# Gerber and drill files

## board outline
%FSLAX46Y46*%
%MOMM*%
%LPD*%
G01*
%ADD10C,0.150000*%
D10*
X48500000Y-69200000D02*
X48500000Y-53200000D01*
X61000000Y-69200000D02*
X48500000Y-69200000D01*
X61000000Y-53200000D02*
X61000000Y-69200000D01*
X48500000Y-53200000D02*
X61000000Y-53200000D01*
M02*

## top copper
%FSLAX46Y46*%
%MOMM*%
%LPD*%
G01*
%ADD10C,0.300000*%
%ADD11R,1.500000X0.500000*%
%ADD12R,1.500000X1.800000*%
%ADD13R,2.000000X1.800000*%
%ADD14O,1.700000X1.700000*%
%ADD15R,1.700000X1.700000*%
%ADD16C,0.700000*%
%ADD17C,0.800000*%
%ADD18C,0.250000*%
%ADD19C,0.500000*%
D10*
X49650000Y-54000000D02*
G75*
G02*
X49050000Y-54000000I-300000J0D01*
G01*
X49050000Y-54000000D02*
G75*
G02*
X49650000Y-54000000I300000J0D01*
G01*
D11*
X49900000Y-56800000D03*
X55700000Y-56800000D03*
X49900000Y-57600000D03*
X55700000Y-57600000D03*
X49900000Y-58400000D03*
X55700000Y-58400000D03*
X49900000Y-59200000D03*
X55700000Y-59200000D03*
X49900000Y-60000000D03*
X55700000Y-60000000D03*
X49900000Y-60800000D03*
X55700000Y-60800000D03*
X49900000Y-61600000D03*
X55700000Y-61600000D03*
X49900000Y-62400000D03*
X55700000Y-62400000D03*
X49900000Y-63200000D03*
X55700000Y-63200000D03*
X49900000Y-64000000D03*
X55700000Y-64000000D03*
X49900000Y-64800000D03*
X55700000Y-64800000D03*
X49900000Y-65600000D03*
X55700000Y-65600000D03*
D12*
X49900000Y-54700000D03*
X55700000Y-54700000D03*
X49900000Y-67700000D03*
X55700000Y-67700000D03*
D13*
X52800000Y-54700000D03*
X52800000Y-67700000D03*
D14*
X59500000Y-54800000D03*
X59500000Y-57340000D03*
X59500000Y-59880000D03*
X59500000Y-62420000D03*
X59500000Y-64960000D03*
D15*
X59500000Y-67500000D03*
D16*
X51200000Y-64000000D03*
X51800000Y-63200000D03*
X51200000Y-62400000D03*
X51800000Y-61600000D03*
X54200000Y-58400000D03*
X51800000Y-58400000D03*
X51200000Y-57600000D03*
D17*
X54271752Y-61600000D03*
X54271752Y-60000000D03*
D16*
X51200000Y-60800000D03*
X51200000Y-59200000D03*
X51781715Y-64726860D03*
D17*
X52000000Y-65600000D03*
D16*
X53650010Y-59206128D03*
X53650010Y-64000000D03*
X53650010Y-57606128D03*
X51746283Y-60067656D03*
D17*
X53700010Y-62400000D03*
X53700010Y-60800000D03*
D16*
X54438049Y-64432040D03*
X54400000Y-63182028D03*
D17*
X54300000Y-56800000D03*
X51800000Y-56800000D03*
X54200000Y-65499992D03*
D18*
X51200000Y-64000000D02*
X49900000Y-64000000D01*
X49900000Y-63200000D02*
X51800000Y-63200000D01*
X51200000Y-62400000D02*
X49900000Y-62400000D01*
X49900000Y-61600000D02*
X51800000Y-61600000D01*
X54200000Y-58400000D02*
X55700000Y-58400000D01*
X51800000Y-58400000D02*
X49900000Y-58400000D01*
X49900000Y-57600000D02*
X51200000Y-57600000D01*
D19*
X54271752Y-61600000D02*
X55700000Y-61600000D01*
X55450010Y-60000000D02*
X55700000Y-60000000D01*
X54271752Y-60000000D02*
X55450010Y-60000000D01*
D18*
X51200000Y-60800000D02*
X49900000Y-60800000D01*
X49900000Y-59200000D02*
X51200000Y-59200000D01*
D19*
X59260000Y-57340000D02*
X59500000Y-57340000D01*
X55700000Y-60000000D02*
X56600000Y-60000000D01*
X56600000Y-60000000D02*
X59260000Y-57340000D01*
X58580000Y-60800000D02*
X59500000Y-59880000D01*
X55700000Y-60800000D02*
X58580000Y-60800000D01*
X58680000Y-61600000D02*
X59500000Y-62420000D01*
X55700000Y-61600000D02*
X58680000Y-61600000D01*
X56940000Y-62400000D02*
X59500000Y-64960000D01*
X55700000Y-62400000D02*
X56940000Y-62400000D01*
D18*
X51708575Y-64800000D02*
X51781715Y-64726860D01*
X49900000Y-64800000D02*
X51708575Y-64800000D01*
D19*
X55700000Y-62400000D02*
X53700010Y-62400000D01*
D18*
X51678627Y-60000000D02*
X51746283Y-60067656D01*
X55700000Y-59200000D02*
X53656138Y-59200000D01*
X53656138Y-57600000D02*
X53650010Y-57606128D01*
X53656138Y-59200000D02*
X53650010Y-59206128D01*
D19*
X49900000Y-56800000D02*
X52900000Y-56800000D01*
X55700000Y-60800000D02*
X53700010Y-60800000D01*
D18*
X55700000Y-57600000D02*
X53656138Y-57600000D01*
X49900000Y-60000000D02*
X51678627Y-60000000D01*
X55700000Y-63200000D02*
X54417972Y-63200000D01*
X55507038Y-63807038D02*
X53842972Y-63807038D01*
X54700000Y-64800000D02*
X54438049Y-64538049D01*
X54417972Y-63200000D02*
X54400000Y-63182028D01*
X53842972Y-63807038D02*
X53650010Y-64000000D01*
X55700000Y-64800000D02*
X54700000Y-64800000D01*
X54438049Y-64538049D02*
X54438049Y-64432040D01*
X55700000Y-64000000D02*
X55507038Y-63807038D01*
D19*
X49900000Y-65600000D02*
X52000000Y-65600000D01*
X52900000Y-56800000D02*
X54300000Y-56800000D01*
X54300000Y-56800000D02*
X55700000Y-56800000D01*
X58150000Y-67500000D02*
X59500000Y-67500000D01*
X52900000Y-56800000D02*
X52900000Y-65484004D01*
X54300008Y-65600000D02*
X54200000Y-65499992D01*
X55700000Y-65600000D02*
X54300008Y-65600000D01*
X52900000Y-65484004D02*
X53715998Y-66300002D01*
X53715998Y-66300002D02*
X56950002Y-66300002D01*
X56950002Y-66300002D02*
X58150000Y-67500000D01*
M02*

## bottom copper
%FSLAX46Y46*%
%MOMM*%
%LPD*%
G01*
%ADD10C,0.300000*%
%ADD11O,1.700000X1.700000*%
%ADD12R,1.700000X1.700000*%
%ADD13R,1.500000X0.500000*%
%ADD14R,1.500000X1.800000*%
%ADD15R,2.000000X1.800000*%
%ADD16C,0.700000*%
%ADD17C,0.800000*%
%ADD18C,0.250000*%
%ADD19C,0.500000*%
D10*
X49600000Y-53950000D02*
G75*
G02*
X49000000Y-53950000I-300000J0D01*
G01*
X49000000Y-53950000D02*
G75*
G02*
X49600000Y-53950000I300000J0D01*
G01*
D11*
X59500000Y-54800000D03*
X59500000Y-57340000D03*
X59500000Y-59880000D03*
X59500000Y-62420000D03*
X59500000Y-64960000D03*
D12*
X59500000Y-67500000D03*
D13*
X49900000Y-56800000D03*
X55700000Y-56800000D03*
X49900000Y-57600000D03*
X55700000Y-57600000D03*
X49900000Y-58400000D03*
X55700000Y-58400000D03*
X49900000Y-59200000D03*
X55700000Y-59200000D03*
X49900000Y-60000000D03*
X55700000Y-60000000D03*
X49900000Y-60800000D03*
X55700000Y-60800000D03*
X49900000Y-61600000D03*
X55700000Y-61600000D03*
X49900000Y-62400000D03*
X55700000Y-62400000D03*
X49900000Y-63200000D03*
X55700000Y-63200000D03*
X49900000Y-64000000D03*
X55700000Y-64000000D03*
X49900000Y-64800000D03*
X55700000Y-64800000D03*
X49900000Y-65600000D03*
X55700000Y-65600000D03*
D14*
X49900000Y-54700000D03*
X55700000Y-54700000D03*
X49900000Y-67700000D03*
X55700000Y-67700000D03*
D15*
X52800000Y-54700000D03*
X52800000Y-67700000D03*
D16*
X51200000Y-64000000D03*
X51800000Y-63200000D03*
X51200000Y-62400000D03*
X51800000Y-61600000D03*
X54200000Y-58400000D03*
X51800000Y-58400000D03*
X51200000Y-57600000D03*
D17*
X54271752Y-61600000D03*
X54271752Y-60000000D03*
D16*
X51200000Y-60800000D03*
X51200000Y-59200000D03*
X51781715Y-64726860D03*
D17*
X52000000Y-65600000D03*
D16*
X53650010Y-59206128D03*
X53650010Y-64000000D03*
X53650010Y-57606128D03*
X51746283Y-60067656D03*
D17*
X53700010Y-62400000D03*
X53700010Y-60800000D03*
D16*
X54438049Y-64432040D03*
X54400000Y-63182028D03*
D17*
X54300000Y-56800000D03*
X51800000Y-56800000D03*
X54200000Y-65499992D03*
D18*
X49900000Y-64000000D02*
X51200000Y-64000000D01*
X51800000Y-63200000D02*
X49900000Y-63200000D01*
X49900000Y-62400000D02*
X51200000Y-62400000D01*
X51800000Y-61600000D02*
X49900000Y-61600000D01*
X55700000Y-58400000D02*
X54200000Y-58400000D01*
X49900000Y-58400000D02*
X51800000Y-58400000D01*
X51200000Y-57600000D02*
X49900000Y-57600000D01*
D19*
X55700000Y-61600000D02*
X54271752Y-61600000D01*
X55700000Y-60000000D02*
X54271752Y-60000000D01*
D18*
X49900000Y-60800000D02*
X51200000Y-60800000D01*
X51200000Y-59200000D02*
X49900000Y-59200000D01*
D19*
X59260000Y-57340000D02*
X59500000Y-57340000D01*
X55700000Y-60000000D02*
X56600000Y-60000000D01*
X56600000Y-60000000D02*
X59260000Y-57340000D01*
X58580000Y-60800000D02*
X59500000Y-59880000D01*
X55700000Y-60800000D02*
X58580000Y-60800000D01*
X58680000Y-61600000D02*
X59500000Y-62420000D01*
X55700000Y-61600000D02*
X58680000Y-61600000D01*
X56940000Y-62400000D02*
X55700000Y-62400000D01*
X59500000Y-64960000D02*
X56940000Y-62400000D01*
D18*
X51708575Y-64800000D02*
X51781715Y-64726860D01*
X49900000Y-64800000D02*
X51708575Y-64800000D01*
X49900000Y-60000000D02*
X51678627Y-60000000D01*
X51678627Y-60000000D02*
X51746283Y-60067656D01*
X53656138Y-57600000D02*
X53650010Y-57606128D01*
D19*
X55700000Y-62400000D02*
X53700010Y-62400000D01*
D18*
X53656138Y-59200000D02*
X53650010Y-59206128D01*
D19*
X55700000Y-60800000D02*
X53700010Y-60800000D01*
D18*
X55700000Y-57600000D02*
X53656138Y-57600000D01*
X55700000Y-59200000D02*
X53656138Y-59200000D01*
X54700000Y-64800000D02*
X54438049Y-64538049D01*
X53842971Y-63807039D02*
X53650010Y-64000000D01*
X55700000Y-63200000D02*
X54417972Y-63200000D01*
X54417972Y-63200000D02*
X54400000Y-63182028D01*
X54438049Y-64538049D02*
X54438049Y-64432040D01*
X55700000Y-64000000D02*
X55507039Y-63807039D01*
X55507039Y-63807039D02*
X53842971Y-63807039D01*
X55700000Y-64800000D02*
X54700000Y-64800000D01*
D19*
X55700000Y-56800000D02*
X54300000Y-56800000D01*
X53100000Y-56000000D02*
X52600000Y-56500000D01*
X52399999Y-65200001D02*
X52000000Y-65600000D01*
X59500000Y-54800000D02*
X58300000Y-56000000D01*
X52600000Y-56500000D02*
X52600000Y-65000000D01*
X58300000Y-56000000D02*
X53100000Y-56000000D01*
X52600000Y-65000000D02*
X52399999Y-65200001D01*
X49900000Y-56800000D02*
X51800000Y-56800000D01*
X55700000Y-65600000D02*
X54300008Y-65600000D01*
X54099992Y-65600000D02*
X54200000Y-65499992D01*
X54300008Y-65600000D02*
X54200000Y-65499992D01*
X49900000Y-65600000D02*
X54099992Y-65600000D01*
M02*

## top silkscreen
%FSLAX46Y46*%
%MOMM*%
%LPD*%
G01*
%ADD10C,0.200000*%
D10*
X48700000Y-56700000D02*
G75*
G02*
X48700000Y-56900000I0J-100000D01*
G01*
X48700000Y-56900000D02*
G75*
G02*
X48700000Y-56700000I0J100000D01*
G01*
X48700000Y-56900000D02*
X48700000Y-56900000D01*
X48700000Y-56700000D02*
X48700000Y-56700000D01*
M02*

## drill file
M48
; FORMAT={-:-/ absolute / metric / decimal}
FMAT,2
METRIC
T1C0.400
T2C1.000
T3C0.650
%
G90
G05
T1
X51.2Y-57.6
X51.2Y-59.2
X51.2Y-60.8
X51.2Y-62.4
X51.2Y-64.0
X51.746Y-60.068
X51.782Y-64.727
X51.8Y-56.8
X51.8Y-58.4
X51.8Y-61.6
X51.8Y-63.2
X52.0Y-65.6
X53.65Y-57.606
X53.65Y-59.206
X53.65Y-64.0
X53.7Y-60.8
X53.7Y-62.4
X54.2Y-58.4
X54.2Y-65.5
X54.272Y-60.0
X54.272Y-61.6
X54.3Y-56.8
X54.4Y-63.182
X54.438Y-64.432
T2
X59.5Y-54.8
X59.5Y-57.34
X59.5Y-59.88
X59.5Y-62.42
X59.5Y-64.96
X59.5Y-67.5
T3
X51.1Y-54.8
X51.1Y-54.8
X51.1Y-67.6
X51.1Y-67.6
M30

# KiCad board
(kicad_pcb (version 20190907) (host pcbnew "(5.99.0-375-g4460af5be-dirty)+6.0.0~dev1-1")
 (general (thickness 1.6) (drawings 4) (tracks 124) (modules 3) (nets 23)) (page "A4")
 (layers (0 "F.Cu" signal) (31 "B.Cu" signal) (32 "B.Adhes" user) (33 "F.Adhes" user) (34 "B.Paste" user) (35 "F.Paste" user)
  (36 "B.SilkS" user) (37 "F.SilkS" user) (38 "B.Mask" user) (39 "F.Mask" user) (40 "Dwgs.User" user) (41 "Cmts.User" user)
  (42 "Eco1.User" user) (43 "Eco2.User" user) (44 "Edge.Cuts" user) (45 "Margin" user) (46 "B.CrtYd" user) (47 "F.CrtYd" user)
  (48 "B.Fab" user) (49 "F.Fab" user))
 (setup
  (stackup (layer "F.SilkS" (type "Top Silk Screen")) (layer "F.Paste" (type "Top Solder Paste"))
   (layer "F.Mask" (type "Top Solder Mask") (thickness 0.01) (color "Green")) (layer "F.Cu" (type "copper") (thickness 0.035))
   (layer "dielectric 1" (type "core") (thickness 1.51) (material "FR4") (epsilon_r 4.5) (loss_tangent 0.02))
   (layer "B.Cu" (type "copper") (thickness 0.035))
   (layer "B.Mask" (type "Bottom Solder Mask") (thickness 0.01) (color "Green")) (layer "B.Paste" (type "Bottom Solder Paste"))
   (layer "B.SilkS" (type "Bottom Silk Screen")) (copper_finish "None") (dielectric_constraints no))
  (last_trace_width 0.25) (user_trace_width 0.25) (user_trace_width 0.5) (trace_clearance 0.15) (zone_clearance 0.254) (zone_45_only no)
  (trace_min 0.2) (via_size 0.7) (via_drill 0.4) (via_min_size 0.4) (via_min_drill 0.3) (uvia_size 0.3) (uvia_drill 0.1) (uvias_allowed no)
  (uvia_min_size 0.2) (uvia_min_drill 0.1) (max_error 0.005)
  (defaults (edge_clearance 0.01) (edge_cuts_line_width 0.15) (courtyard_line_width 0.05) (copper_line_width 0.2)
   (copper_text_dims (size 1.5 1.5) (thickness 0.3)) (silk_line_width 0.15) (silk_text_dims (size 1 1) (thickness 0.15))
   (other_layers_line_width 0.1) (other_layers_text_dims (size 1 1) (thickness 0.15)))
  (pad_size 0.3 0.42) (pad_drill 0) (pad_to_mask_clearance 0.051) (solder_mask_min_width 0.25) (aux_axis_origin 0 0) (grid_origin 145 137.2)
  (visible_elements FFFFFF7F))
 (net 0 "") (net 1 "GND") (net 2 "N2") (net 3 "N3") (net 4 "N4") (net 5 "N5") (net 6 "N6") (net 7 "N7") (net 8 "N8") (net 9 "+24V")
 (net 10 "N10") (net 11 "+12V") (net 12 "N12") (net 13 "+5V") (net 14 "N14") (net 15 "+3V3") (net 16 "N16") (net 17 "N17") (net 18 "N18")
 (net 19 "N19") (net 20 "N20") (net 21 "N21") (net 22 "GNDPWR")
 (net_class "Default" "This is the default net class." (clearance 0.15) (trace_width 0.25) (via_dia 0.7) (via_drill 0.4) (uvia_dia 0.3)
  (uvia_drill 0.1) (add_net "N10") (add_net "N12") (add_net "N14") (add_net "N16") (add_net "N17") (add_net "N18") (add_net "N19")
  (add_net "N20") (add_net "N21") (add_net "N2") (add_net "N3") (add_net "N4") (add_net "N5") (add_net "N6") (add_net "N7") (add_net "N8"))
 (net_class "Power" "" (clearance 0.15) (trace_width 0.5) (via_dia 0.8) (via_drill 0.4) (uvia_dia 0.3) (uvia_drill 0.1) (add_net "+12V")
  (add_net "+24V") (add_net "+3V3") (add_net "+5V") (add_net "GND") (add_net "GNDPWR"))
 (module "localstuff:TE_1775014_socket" (layer "F.Cu") (at 52.8 61.2 -90)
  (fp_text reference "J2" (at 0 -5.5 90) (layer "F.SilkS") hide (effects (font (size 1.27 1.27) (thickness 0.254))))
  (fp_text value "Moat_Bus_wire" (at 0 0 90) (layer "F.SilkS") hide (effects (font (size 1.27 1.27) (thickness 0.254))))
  (fp_arc (start -4.4 4.1) (end -4.3 4.1) (angle -180) (layer "F.SilkS") (width 0.2))
  (fp_arc (start -4.4 4.1) (end -4.5 4.1) (angle -180) (layer "F.SilkS") (width 0.2))
  (fp_line (start -4.3 4.1) (end -4.3 4.1) (layer "F.SilkS") (width 0.2))
  (fp_line (start -4.5 4.1) (end -4.5 4.1) (layer "F.SilkS") (width 0.2))
  (fp_circle (center -7.2 3.45) (end -6.9 3.45) (layer "F.Cu") (width 0.3))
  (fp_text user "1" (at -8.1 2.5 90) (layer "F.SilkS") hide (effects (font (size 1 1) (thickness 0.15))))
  (pad "1" smd rect (at -4.4 2.9 270) (size 0.5 1.5) (layers "F.Cu" "F.Paste" "F.Mask") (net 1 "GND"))
  (pad "2" smd rect (at -4.4 -2.9 270) (size 0.5 1.5) (layers "F.Cu" "F.Paste" "F.Mask") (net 1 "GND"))
  (pad "3" smd rect (at -3.6 2.9 270) (size 0.5 1.5) (layers "F.Cu" "F.Paste" "F.Mask") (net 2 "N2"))
  (pad "4" smd rect (at -3.6 -2.9 270) (size 0.5 1.5) (layers "F.Cu" "F.Paste" "F.Mask") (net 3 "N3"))
  (pad "5" smd rect (at -2.8 2.9 270) (size 0.5 1.5) (layers "F.Cu" "F.Paste" "F.Mask") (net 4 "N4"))
  (pad "6" smd rect (at -2.8 -2.9 270) (size 0.5 1.5) (layers "F.Cu" "F.Paste" "F.Mask") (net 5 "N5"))
  (pad "7" smd rect (at -2 2.9 270) (size 0.5 1.5) (layers "F.Cu" "F.Paste" "F.Mask") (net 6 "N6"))
  (pad "8" smd rect (at -2 -2.9 270) (size 0.5 1.5) (layers "F.Cu" "F.Paste" "F.Mask") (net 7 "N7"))
  (pad "9" smd rect (at -1.2 2.9 270) (size 0.5 1.5) (layers "F.Cu" "F.Paste" "F.Mask") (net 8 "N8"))
  (pad "10" smd rect (at -1.2 -2.9 270) (size 0.5 1.5) (layers "F.Cu" "F.Paste" "F.Mask") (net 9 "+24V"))
  (pad "11" smd rect (at -0.4 2.9 270) (size 0.5 1.5) (layers "F.Cu" "F.Paste" "F.Mask") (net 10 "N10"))
  (pad "12" smd rect (at -0.4 -2.9 270) (size 0.5 1.5) (layers "F.Cu" "F.Paste" "F.Mask") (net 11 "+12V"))
  (pad "13" smd rect (at 0.4 2.9 270) (size 0.5 1.5) (layers "F.Cu" "F.Paste" "F.Mask") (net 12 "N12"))
  (pad "14" smd rect (at 0.4 -2.9 270) (size 0.5 1.5) (layers "F.Cu" "F.Paste" "F.Mask") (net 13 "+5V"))
  (pad "15" smd rect (at 1.2 2.9 270) (size 0.5 1.5) (layers "F.Cu" "F.Paste" "F.Mask") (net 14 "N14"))
  (pad "16" smd rect (at 1.2 -2.9 270) (size 0.5 1.5) (layers "F.Cu" "F.Paste" "F.Mask") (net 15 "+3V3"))
  (pad "17" smd rect (at 2 2.9 270) (size 0.5 1.5) (layers "F.Cu" "F.Paste" "F.Mask") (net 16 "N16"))
  (pad "18" smd rect (at 2 -2.9 270) (size 0.5 1.5) (layers "F.Cu" "F.Paste" "F.Mask") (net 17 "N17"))
  (pad "19" smd rect (at 2.8 2.9 270) (size 0.5 1.5) (layers "F.Cu" "F.Paste" "F.Mask") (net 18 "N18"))
  (pad "20" smd rect (at 2.8 -2.9 270) (size 0.5 1.5) (layers "F.Cu" "F.Paste" "F.Mask") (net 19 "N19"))
  (pad "21" smd rect (at 3.6 2.9 270) (size 0.5 1.5) (layers "F.Cu" "F.Paste" "F.Mask") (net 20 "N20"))
  (pad "22" smd rect (at 3.6 -2.9 270) (size 0.5 1.5) (layers "F.Cu" "F.Paste" "F.Mask") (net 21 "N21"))
  (pad "23" smd rect (at 4.4 2.9 270) (size 0.5 1.5) (layers "F.Cu" "F.Paste" "F.Mask") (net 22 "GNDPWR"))
  (pad "24" smd rect (at 4.4 -2.9 270) (size 0.5 1.5) (layers "F.Cu" "F.Paste" "F.Mask") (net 22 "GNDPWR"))
  (pad "MNT" smd rect (at -6.5 2.9) (size 1.5 1.8) (layers "F.Cu" "F.Paste" "F.Mask") (solder_paste_margin -0.05) (clearance 0.001))
  (pad "MNT" smd rect (at -6.5 -2.9) (size 1.5 1.8) (layers "F.Cu" "F.Paste" "F.Mask"))
  (pad "MNT" smd rect (at 6.5 2.9) (size 1.5 1.8) (layers "F.Cu" "F.Paste" "F.Mask") (solder_paste_margin -0.05) (clearance 0.001))
  (pad "MNT" smd rect (at 6.5 -2.9) (size 1.5 1.8) (layers "F.Cu" "F.Paste" "F.Mask"))
  (pad "MNT" smd rect (at -6.5 0 270) (size 1.8 2) (layers "F.Cu" "F.Paste" "F.Mask"))
  (pad "MNT" smd rect (at 6.5 0 270) (size 1.8 2) (layers "F.Cu" "F.Paste" "F.Mask"))
  (pad "" np_thru_hole circle (at -6.4 1.7 270) (size 0.65 0.65) (drill 0.65) (layers *.Cu *.Mask) (clearance 0.01))
  (pad "" np_thru_hole circle (at 6.4 1.7 270) (size 0.65 0.65) (drill 0.65) (layers *.Cu *.Mask) (clearance 0.0001)))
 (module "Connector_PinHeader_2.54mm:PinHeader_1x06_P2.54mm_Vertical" (layer "B.Cu") (at 59.5 67.5)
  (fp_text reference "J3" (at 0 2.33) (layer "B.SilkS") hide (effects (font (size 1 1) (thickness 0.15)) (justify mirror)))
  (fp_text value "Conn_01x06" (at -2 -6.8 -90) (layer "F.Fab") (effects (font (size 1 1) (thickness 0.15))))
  (pad "6" thru_hole oval (at 0 -12.7) (size 1.7 1.7) (drill 1) (layers *.Cu *.Mask) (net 22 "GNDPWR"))
  (pad "5" thru_hole oval (at 0 -10.16) (size 1.7 1.7) (drill 1) (layers *.Cu *.Mask) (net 9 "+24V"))
  (pad "4" thru_hole oval (at 0 -7.62) (size 1.7 1.7) (drill 1) (layers *.Cu *.Mask) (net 11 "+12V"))
  (pad "3" thru_hole oval (at 0 -5.08) (size 1.7 1.7) (drill 1) (layers *.Cu *.Mask) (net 13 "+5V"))
  (pad "2" thru_hole oval (at 0 -2.54) (size 1.7 1.7) (drill 1) (layers *.Cu *.Mask) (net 15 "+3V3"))
  (pad "1" thru_hole rect (at 0 0) (size 1.7 1.7) (drill 1) (layers *.Cu *.Mask) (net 1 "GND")))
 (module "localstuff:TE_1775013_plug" (layer "B.Cu") (at 52.8 61.2 90)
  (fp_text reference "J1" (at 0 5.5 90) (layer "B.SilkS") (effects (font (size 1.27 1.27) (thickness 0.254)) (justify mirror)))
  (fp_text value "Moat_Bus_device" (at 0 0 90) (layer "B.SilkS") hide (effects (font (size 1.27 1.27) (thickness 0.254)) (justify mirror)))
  (fp_circle (center 7.25 -3.5) (end 7.55 -3.5) (layer "B.Cu") (width 0.3))
  (pad "1" smd rect (at 4.4 -2.9 90) (size 0.5 1.5) (layers "B.Cu" "B.Paste" "B.Mask") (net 1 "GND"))
  (pad "2" smd rect (at 4.4 2.9 90) (size 0.5 1.5) (layers "B.Cu" "B.Paste" "B.Mask") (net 1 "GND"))
  (pad "3" smd rect (at 3.6 -2.9 90) (size 0.5 1.5) (layers "B.Cu" "B.Paste" "B.Mask") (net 2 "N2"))
  (pad "4" smd rect (at 3.6 2.9 90) (size 0.5 1.5) (layers "B.Cu" "B.Paste" "B.Mask") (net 3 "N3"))
  (pad "5" smd rect (at 2.8 -2.9 90) (size 0.5 1.5) (layers "B.Cu" "B.Paste" "B.Mask") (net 4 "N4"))
  (pad "6" smd rect (at 2.8 2.9 90) (size 0.5 1.5) (layers "B.Cu" "B.Paste" "B.Mask") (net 5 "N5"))
  (pad "7" smd rect (at 2 -2.9 90) (size 0.5 1.5) (layers "B.Cu" "B.Paste" "B.Mask") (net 6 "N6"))
  (pad "8" smd rect (at 2 2.9 90) (size 0.5 1.5) (layers "B.Cu" "B.Paste" "B.Mask") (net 7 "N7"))
  (pad "9" smd rect (at 1.2 -2.9 90) (size 0.5 1.5) (layers "B.Cu" "B.Paste" "B.Mask") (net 8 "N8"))
  (pad "10" smd rect (at 1.2 2.9 90) (size 0.5 1.5) (layers "B.Cu" "B.Paste" "B.Mask") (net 9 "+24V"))
  (pad "11" smd rect (at 0.4 -2.9 90) (size 0.5 1.5) (layers "B.Cu" "B.Paste" "B.Mask") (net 10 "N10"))
  (pad "12" smd rect (at 0.4 2.9 90) (size 0.5 1.5) (layers "B.Cu" "B.Paste" "B.Mask") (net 11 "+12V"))
  (pad "13" smd rect (at -0.4 -2.9 90) (size 0.5 1.5) (layers "B.Cu" "B.Paste" "B.Mask") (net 12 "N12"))
  (pad "14" smd rect (at -0.4 2.9 90) (size 0.5 1.5) (layers "B.Cu" "B.Paste" "B.Mask") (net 13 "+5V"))
  (pad "15" smd rect (at -1.2 -2.9 90) (size 0.5 1.5) (layers "B.Cu" "B.Paste" "B.Mask") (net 14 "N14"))
  (pad "16" smd rect (at -1.2 2.9 90) (size 0.5 1.5) (layers "B.Cu" "B.Paste" "B.Mask") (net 15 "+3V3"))
  (pad "17" smd rect (at -2 -2.9 90) (size 0.5 1.5) (layers "B.Cu" "B.Paste" "B.Mask") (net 16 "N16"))
  (pad "18" smd rect (at -2 2.9 90) (size 0.5 1.5) (layers "B.Cu" "B.Paste" "B.Mask") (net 17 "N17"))
  (pad "19" smd rect (at -2.8 -2.9 90) (size 0.5 1.5) (layers "B.Cu" "B.Paste" "B.Mask") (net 18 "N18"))
  (pad "20" smd rect (at -2.8 2.9 90) (size 0.5 1.5) (layers "B.Cu" "B.Paste" "B.Mask") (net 19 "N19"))
  (pad "21" smd rect (at -3.6 -2.9 90) (size 0.5 1.5) (layers "B.Cu" "B.Paste" "B.Mask") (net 20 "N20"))
  (pad "22" smd rect (at -3.6 2.9 90) (size 0.5 1.5) (layers "B.Cu" "B.Paste" "B.Mask") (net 21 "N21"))
  (pad "23" smd rect (at -4.4 -2.9 90) (size 0.5 1.5) (layers "B.Cu" "B.Paste" "B.Mask") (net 22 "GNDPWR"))
  (pad "24" smd rect (at -4.4 2.9 90) (size 0.5 1.5) (layers "B.Cu" "B.Paste" "B.Mask") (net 22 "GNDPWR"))
  (pad "MNT" smd rect (at 6.5 -2.9 180) (size 1.5 1.8) (layers "B.Cu" "B.Paste" "B.Mask"))
  (pad "MNT" smd rect (at 6.5 2.9 180) (size 1.5 1.8) (layers "B.Cu" "B.Paste" "B.Mask"))
  (pad "MNT" smd rect (at -6.5 -2.9 180) (size 1.5 1.8) (layers "B.Cu" "B.Paste" "B.Mask"))
  (pad "MNT" smd rect (at -6.5 2.9 180) (size 1.5 1.8) (layers "B.Cu" "B.Paste" "B.Mask"))
  (pad "MNT" smd rect (at 6.5 0 90) (size 1.8 2) (layers "B.Cu" "B.Paste" "B.Mask"))
  (pad "MNT" smd rect (at -6.5 0 90) (size 1.8 2) (layers "B.Cu" "B.Paste" "B.Mask"))
  (pad "" np_thru_hole circle (at 6.4 -1.7 90) (size 0.65 0.65) (drill 0.65) (layers *.Cu *.Mask))
  (pad "" np_thru_hole circle (at -6.4 -1.7 90) (size 0.65 0.65) (drill 0.65) (layers *.Cu *.Mask)))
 (gr_line (start 48.5 69.2) (end 48.5 53.2) (layer "Edge.Cuts") (width 0.15))
 (gr_line (start 61 69.2) (end 48.5 69.2) (layer "Edge.Cuts") (width 0.15))
 (gr_line (start 61 53.2) (end 61 69.2) (layer "Edge.Cuts") (width 0.15))
 (gr_line (start 48.5 53.2) (end 61 53.2) (layer "Edge.Cuts") (width 0.15))
 (segment (start 51.2 64) (end 49.9 64) (width 0.25) (layer "F.Cu") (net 18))
 (segment (start 49.9 64) (end 51.2 64) (width 0.25) (layer "B.Cu") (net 18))
 (via (at 51.2 64) (size 0.7) (drill 0.4) (layers "F.Cu" "B.Cu") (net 18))
 (segment (start 51.8 63.2) (end 49.9 63.2) (width 0.25) (layer "B.Cu") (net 16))
 (segment (start 49.9 63.2) (end 51.8 63.2) (width 0.25) (layer "F.Cu") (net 16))
 (via (at 51.8 63.2) (size 0.7) (drill 0.4) (layers "F.Cu" "B.Cu") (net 16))
 (segment (start 51.2 62.4) (end 49.9 62.4) (width 0.25) (layer "F.Cu") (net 14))
 (segment (start 49.9 62.4) (end 51.2 62.4) (width 0.25) (layer "B.Cu") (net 14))
 (via (at 51.2 62.4) (size 0.7) (drill 0.4) (layers "F.Cu" "B.Cu") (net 14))
 (segment (start 51.8 61.6) (end 49.9 61.6) (width 0.25) (layer "B.Cu") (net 12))
 (segment (start 49.9 61.6) (end 51.8 61.6) (width 0.25) (layer "F.Cu") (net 12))
 (via (at 51.8 61.6) (size 0.7) (drill 0.4) (layers "F.Cu" "B.Cu") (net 12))
 (segment (start 54.2 58.4) (end 55.7 58.4) (width 0.25) (layer "F.Cu") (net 5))
 (segment (start 55.7 58.4) (end 54.2 58.4) (width 0.25) (layer "B.Cu") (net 5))
 (via (at 54.2 58.4) (size 0.7) (drill 0.4) (layers "F.Cu" "B.Cu") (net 5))
 (segment (start 51.8 58.4) (end 49.9 58.4) (width 0.25) (layer "F.Cu") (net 4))
 (segment (start 49.9 58.4) (end 51.8 58.4) (width 0.25) (layer "B.Cu") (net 4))
 (via (at 51.8 58.4) (size 0.7) (drill 0.4) (layers "F.Cu" "B.Cu") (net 4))
 (segment (start 51.2 57.6) (end 49.9 57.6) (width 0.25) (layer "B.Cu") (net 2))
 (segment (start 49.9 57.6) (end 51.2 57.6) (width 0.25) (layer "F.Cu") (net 2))
 (via (at 51.2 57.6) (size 0.7) (drill 0.4) (layers "F.Cu" "B.Cu") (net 2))
 (segment (start 54.271752 61.6) (end 55.7 61.6) (width 0.5) (layer "F.Cu") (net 13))
 (segment (start 55.7 61.6) (end 54.271752 61.6) (width 0.5) (layer "B.Cu") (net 13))
 (via (at 54.271752 61.6) (size 0.8) (drill 0.4) (layers "F.Cu" "B.Cu") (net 13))
 (segment (start 55.45001 60) (end 55.7 60) (width 0.5) (layer "F.Cu") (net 9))
 (segment (start 54.271752 60) (end 55.45001 60) (width 0.5) (layer "F.Cu") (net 9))
 (segment (start 55.7 60) (end 54.271752 60) (width 0.5) (layer "B.Cu") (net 9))
 (via (at 54.271752 60) (size 0.8) (drill 0.4) (layers "F.Cu" "B.Cu") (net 9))
 (segment (start 51.2 60.8) (end 49.9 60.8) (width 0.25) (layer "F.Cu") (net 10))
 (segment (start 49.9 60.8) (end 51.2 60.8) (width 0.25) (layer "B.Cu") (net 10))
 (via (at 51.2 60.8) (size 0.7) (drill 0.4) (layers "F.Cu" "B.Cu") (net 10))
 (segment (start 51.2 59.2) (end 49.9 59.2) (width 0.25) (layer "B.Cu") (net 6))
 (segment (start 49.9 59.2) (end 51.2 59.2) (width 0.25) (layer "F.Cu") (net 6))
 (via (at 51.2 59.2) (size 0.7) (drill 0.4) (layers "F.Cu" "B.Cu") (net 6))
 (segment (start 59.26 57.34) (end 59.5 57.34) (width 0.5) (layer "B.Cu") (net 9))
 (segment (start 55.7 60) (end 56.6 60) (width 0.5) (layer "B.Cu") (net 9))
 (segment (start 56.6 60) (end 59.26 57.34) (width 0.5) (layer "B.Cu") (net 9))
 (segment (start 58.58 60.8) (end 59.5 59.88) (width 0.5) (layer "B.Cu") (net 11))
 (segment (start 55.7 60.8) (end 58.58 60.8) (width 0.5) (layer "B.Cu") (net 11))
 (segment (start 58.68 61.6) (end 59.5 62.42) (width 0.5) (layer "B.Cu") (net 13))
 (segment (start 55.7 61.6) (end 58.68 61.6) (width 0.5) (layer "B.Cu") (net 13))
 (segment (start 56.94 62.4) (end 55.7 62.4) (width 0.5) (layer "B.Cu") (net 15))
 (segment (start 59.5 64.96) (end 56.94 62.4) (width 0.5) (layer "B.Cu") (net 15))
 (segment (start 59.26 57.34) (end 59.5 57.34) (width 0.5) (layer "F.Cu") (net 9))
 (segment (start 55.7 60) (end 56.6 60) (width 0.5) (layer "F.Cu") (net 9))
 (segment (start 56.6 60) (end 59.26 57.34) (width 0.5) (layer "F.Cu") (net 9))
 (segment (start 58.58 60.8) (end 59.5 59.88) (width 0.5) (layer "F.Cu") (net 11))
 (segment (start 55.7 60.8) (end 58.58 60.8) (width 0.5) (layer "F.Cu") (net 11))
 (segment (start 58.68 61.6) (end 59.5 62.42) (width 0.5) (layer "F.Cu") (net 13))
 (segment (start 55.7 61.6) (end 58.68 61.6) (width 0.5) (layer "F.Cu") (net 13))
 (segment (start 56.94 62.4) (end 59.5 64.96) (width 0.5) (layer "F.Cu") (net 15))
 (segment (start 55.7 62.4) (end 56.94 62.4) (width 0.5) (layer "F.Cu") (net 15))
 (via (at 51.781715 64.72686) (size 0.7) (drill 0.4) (layers "F.Cu" "B.Cu") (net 20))
 (segment (start 51.708575 64.8) (end 51.781715 64.72686) (width 0.25) (layer "B.Cu") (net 20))
 (segment (start 51.708575 64.8) (end 51.781715 64.72686) (width 0.25) (layer "F.Cu") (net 20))
 (segment (start 49.9 64.8) (end 51.708575 64.8) (width 0.25) (layer "B.Cu") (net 20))
 (via (at 52 65.6) (size 0.8) (drill 0.4) (layers "F.Cu" "B.Cu") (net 22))
 (segment (start 49.9 64.8) (end 51.708575 64.8) (width 0.25) (layer "F.Cu") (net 20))
 (via (at 53.65001 59.206128) (size 0.7) (drill 0.4) (layers "F.Cu" "B.Cu") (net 7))
 (segment (start 55.7 62.4) (end 53.70001 62.4) (width 0.5) (layer "F.Cu") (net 15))
 (segment (start 49.9 60) (end 51.678627 60) (width 0.25) (layer "B.Cu") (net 8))
 (segment (start 51.678627 60) (end 51.746283 60.067656) (width 0.25) (layer "B.Cu") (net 8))
 (segment (start 51.678627 60) (end 51.746283 60.067656) (width 0.25) (layer "F.Cu") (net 8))
 (segment (start 55.7 59.2) (end 53.656138 59.2) (width 0.25) (layer "F.Cu") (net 7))
 (via (at 53.65001 64) (size 0.7) (drill 0.4) (layers "F.Cu" "B.Cu") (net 19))
 (segment (start 53.656138 57.6) (end 53.65001 57.606128) (width 0.25) (layer "B.Cu") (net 3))
 (segment (start 55.7 62.4) (end 53.70001 62.4) (width 0.5) (layer "B.Cu") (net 15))
 (segment (start 53.656138 59.2) (end 53.65001 59.206128) (width 0.25) (layer "B.Cu") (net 7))
 (segment (start 55.7 60.8) (end 53.70001 60.8) (width 0.5) (layer "B.Cu") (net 11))
 (segment (start 53.656138 57.6) (end 53.65001 57.606128) (width 0.25) (layer "F.Cu") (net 3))
 (via (at 53.65001 57.606128) (size 0.7) (drill 0.4) (layers "F.Cu" "B.Cu") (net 3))
 (segment (start 53.656138 59.2) (end 53.65001 59.206128) (width 0.25) (layer "F.Cu") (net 7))
 (via (at 51.746283 60.067656) (size 0.7) (drill 0.4) (layers "F.Cu" "B.Cu") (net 8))
 (segment (start 49.9 56.8) (end 52.9 56.8) (width 0.5) (layer "F.Cu") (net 1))
 (segment (start 55.7 60.8) (end 53.70001 60.8) (width 0.5) (layer "F.Cu") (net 11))
 (segment (start 55.7 57.6) (end 53.656138 57.6) (width 0.25) (layer "B.Cu") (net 3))
 (via (at 53.70001 62.4) (size 0.8) (drill 0.4) (layers "F.Cu" "B.Cu") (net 15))
 (via (at 53.70001 60.8) (size 0.8) (drill 0.4) (layers "F.Cu" "B.Cu") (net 11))
 (segment (start 55.7 57.6) (end 53.656138 57.6) (width 0.25) (layer "F.Cu") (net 3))
 (segment (start 55.7 59.2) (end 53.656138 59.2) (width 0.25) (layer "B.Cu") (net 7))
 (segment (start 49.9 60) (end 51.678627 60) (width 0.25) (layer "F.Cu") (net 8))
 (segment (start 55.7 63.2) (end 54.417972 63.2) (width 0.25) (layer "F.Cu") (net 17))
 (segment (start 55.507038 63.807038) (end 53.842972 63.807038) (width 0.25) (layer "F.Cu") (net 19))
 (segment (start 54.7 64.8) (end 54.438049 64.538049) (width 0.25) (layer "B.Cu") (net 21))
 (via (at 54.438049 64.43204) (size 0.7) (drill 0.4) (layers "F.Cu" "B.Cu") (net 21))
 (segment (start 53.842971 63.807039) (end 53.65001 64) (width 0.25) (layer "B.Cu") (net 19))
 (segment (start 54.7 64.8) (end 54.438049 64.538049) (width 0.25) (layer "F.Cu") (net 21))
 (segment (start 55.7 63.2) (end 54.417972 63.2) (width 0.25) (layer "B.Cu") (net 17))
 (segment (start 54.417972 63.2) (end 54.4 63.182028) (width 0.25) (layer "B.Cu") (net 17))
 (segment (start 54.417972 63.2) (end 54.4 63.182028) (width 0.25) (layer "F.Cu") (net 17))
 (segment (start 54.438049 64.538049) (end 54.438049 64.43204) (width 0.25) (layer "B.Cu") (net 21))
 (segment (start 53.842972 63.807038) (end 53.65001 64) (width 0.25) (layer "F.Cu") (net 19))
 (segment (start 55.7 64) (end 55.507039 63.807039) (width 0.25) (layer "B.Cu") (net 19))
 (segment (start 55.507039 63.807039) (end 53.842971 63.807039) (width 0.25) (layer "B.Cu") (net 19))
 (segment (start 55.7 64.8) (end 54.7 64.8) (width 0.25) (layer "F.Cu") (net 21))
 (segment (start 55.7 64.8) (end 54.7 64.8) (width 0.25) (layer "B.Cu") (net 21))
 (segment (start 54.438049 64.538049) (end 54.438049 64.43204) (width 0.25) (layer "F.Cu") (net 21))
 (via (at 54.4 63.182028) (size 0.7) (drill 0.4) (layers "F.Cu" "B.Cu") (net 17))
 (segment (start 55.7 64) (end 55.507038 63.807038) (width 0.25) (layer "F.Cu") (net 19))
 (segment (start 49.9 65.6) (end 52 65.6) (width 0.5) (layer "F.Cu") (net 22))
 (via (at 54.3 56.8) (size 0.8) (drill 0.4) (layers "F.Cu" "B.Cu") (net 1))
 (segment (start 55.7 56.8) (end 54.3 56.8) (width 0.5) (layer "B.Cu") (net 1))
 (segment (start 52.9 56.8) (end 54.3 56.8) (width 0.5) (layer "F.Cu") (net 1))
 (segment (start 53.1 56) (end 52.6 56.5) (width 0.5) (layer "B.Cu") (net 22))
 (segment (start 52.399999 65.200001) (end 52 65.6) (width 0.5) (layer "B.Cu") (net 22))
 (segment (start 59.5 54.8) (end 58.3 56) (width 0.5) (layer "B.Cu") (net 22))
 (segment (start 52.6 56.5) (end 52.6 65) (width 0.5) (layer "B.Cu") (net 22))
 (segment (start 54.3 56.8) (end 55.7 56.8) (width 0.5) (layer "F.Cu") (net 1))
 (segment (start 58.3 56) (end 53.1 56) (width 0.5) (layer "B.Cu") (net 22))
 (segment (start 52.6 65) (end 52.399999 65.200001) (width 0.5) (layer "B.Cu") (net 22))
 (via (at 51.8 56.8) (size 0.8) (drill 0.4) (layers "F.Cu" "B.Cu") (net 1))
 (segment (start 49.9 56.8) (end 51.8 56.8) (width 0.5) (layer "B.Cu") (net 1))
 (segment (start 58.15 67.5) (end 59.5 67.5) (width 0.5) (layer "F.Cu") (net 1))
 (segment (start 55.7 65.6) (end 54.300008 65.6) (width 0.5) (layer "B.Cu") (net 22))
 (segment (start 52.9 56.8) (end 52.9 65.484004) (width 0.5) (layer "F.Cu") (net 1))
 (segment (start 54.300008 65.6) (end 54.2 65.499992) (width 0.5) (layer "F.Cu") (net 22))
 (segment (start 54.099992 65.6) (end 54.2 65.499992) (width 0.5) (layer "B.Cu") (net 22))
 (segment (start 54.300008 65.6) (end 54.2 65.499992) (width 0.5) (layer "B.Cu") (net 22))
 (segment (start 55.7 65.6) (end 54.300008 65.6) (width 0.5) (layer "F.Cu") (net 22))
 (via (at 54.2 65.499992) (size 0.8) (drill 0.4) (layers "F.Cu" "B.Cu") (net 22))
 (segment (start 52.9 65.484004) (end 53.715998 66.300002) (width 0.5) (layer "F.Cu") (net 1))
 (segment (start 49.9 65.6) (end 54.099992 65.6) (width 0.5) (layer "B.Cu") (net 22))
 (segment (start 53.715998 66.300002) (end 56.950002 66.300002) (width 0.5) (layer "F.Cu") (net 1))
 (segment (start 56.950002 66.300002) (end 58.15 67.5) (width 0.5) (layer "F.Cu") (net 1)))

